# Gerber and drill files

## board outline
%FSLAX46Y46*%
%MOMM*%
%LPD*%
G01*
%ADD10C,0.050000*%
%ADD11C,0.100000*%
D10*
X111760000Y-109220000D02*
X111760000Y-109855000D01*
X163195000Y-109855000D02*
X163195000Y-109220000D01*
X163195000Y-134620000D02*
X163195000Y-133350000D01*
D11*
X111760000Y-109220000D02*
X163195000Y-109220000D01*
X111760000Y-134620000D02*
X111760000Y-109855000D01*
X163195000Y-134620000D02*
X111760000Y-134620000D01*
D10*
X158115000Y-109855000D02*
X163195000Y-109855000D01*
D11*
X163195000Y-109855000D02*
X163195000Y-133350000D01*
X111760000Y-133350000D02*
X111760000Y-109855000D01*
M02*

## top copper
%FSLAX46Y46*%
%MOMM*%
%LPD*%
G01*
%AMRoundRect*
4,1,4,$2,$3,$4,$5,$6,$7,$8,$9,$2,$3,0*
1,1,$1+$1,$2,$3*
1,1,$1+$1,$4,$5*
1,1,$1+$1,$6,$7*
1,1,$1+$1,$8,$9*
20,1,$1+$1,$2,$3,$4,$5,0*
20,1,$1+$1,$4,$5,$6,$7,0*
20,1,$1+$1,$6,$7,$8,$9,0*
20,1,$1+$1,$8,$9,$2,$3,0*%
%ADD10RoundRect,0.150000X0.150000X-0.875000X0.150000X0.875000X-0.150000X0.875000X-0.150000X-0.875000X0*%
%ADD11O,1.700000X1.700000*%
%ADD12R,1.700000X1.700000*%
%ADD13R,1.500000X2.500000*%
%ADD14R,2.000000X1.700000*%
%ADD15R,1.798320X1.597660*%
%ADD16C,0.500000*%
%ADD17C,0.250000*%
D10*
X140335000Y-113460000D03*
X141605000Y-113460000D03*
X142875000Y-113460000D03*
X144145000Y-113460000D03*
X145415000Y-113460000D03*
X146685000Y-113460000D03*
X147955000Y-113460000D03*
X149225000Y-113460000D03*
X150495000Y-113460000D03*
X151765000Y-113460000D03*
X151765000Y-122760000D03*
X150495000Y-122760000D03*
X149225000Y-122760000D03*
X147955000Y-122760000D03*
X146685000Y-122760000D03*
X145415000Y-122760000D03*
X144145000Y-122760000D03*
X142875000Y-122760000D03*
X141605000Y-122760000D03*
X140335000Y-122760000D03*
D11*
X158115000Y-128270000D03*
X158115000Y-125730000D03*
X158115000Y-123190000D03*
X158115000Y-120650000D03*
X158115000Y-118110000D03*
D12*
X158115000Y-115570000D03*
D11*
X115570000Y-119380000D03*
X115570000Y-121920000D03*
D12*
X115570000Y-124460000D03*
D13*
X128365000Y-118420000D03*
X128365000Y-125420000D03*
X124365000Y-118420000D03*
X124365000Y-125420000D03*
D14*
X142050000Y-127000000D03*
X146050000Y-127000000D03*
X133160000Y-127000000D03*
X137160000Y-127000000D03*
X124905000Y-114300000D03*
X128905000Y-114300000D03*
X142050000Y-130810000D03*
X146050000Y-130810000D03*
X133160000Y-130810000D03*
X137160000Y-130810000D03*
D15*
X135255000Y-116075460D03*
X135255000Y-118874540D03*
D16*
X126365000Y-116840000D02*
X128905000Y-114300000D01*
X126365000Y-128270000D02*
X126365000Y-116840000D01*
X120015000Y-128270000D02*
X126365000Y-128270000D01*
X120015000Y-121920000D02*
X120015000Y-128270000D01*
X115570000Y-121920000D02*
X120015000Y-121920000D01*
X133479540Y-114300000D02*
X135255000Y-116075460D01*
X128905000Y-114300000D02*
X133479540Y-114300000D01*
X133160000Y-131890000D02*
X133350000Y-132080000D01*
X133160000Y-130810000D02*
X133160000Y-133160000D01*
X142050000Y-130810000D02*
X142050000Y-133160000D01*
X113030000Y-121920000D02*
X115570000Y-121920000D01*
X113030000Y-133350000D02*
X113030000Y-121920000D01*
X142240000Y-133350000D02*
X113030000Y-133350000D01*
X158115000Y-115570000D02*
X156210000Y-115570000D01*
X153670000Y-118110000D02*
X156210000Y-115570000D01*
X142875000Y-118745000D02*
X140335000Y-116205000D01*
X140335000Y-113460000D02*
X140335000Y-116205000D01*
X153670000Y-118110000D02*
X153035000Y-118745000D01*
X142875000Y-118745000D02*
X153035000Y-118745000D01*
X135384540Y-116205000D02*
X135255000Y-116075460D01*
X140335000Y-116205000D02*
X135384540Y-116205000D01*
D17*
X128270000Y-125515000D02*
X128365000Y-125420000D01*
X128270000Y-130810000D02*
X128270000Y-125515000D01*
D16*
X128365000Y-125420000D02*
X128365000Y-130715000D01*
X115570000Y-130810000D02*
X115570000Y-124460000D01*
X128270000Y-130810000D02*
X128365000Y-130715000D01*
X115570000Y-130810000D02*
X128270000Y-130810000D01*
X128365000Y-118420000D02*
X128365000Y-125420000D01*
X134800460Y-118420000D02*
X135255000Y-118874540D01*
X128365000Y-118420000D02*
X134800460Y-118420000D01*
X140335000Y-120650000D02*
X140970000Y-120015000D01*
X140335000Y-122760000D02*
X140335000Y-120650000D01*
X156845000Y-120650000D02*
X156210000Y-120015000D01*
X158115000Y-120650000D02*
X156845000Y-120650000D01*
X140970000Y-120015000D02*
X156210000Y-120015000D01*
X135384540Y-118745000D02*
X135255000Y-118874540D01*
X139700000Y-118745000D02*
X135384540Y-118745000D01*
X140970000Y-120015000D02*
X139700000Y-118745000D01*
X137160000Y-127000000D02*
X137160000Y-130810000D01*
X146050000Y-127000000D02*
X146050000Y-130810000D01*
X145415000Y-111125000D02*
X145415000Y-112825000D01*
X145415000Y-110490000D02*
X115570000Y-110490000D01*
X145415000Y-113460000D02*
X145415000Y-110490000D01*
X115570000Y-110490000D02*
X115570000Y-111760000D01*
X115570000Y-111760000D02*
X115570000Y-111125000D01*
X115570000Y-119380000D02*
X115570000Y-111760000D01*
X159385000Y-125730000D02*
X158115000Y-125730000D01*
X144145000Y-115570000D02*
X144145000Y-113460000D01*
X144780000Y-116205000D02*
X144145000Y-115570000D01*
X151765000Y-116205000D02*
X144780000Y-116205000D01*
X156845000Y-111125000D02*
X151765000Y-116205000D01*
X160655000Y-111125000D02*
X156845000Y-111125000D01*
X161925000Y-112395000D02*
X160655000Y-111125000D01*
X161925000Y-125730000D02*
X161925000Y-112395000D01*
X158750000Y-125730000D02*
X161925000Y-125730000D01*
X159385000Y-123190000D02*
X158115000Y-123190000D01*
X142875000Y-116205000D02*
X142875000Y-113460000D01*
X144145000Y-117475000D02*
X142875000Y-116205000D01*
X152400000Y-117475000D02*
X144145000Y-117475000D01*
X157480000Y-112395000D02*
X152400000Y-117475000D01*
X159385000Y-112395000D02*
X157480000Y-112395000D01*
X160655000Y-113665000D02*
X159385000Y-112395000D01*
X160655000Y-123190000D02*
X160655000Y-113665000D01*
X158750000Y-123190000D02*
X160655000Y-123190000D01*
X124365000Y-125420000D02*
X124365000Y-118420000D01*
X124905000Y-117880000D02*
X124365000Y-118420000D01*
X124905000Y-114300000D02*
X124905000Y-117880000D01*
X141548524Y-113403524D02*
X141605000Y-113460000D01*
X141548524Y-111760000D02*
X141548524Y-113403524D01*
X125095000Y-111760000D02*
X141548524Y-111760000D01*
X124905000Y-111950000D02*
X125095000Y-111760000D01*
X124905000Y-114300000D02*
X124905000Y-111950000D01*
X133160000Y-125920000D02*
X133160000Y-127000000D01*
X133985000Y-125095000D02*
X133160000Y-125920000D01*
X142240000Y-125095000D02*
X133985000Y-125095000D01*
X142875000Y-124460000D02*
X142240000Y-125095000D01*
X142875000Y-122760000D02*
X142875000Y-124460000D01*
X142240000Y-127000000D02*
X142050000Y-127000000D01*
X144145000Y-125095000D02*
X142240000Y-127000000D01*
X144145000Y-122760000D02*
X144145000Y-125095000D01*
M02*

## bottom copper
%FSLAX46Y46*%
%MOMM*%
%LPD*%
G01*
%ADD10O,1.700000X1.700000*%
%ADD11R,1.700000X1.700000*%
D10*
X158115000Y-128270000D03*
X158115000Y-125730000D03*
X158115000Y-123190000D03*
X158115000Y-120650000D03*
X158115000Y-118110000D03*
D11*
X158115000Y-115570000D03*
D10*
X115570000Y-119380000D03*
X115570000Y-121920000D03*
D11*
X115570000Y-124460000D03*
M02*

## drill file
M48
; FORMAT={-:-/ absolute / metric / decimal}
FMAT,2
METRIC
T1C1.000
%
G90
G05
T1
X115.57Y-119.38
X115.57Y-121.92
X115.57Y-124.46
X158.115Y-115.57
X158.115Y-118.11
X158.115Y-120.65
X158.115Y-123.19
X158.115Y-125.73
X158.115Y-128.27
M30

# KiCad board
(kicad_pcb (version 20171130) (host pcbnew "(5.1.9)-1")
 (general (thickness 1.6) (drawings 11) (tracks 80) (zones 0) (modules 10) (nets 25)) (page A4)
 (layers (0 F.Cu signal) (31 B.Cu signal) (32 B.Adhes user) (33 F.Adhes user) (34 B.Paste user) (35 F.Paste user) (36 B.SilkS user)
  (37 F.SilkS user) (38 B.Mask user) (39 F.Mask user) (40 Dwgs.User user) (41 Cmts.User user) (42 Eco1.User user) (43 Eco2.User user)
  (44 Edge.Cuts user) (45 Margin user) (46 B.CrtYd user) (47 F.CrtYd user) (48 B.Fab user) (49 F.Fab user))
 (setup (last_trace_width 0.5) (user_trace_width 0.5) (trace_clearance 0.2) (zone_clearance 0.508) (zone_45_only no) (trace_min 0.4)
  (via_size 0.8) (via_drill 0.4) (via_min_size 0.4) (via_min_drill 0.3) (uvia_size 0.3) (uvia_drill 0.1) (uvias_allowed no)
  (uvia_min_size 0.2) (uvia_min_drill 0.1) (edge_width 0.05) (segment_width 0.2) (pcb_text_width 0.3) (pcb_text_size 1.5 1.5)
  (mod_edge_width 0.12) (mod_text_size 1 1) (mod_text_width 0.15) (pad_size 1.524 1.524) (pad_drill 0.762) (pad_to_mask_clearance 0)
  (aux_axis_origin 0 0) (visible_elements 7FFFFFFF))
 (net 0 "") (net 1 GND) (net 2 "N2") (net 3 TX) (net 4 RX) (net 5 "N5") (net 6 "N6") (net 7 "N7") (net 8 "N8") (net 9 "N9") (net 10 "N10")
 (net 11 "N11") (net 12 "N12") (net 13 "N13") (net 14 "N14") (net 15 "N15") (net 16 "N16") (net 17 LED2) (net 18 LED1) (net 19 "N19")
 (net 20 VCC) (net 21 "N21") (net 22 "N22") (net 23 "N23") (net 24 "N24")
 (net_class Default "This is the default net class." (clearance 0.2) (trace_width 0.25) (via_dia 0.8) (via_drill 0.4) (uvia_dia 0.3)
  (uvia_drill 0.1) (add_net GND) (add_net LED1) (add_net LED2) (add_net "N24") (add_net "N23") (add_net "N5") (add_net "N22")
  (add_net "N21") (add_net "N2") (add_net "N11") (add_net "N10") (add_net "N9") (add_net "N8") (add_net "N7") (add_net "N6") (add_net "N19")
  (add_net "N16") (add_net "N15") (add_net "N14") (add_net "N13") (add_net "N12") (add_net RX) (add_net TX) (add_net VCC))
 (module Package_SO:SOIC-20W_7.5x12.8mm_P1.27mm (layer F.Cu) (at 146.05 118.11 90)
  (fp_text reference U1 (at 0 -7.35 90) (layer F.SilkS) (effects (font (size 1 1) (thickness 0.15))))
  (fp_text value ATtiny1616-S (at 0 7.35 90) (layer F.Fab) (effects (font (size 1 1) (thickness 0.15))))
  (pad 20 smd roundrect (at 4.65 -5.715 90) (size 2.05 0.6) (layers F.Cu F.Paste F.Mask) (roundrect_rratio 0.25) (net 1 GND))
  (pad 19 smd roundrect (at 4.65 -4.445 90) (size 2.05 0.6) (layers F.Cu F.Paste F.Mask) (roundrect_rratio 0.25) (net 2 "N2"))
  (pad 18 smd roundrect (at 4.65 -3.175 90) (size 2.05 0.6) (layers F.Cu F.Paste F.Mask) (roundrect_rratio 0.25) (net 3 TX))
  (pad 17 smd roundrect (at 4.65 -1.905 90) (size 2.05 0.6) (layers F.Cu F.Paste F.Mask) (roundrect_rratio 0.25) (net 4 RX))
  (pad 16 smd roundrect (at 4.65 -0.635 90) (size 2.05 0.6) (layers F.Cu F.Paste F.Mask) (roundrect_rratio 0.25) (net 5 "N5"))
  (pad 15 smd roundrect (at 4.65 0.635 90) (size 2.05 0.6) (layers F.Cu F.Paste F.Mask) (roundrect_rratio 0.25) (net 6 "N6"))
  (pad 14 smd roundrect (at 4.65 1.905 90) (size 2.05 0.6) (layers F.Cu F.Paste F.Mask) (roundrect_rratio 0.25) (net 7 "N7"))
  (pad 13 smd roundrect (at 4.65 3.175 90) (size 2.05 0.6) (layers F.Cu F.Paste F.Mask) (roundrect_rratio 0.25) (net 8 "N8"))
  (pad 12 smd roundrect (at 4.65 4.445 90) (size 2.05 0.6) (layers F.Cu F.Paste F.Mask) (roundrect_rratio 0.25) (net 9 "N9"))
  (pad 11 smd roundrect (at 4.65 5.715 90) (size 2.05 0.6) (layers F.Cu F.Paste F.Mask) (roundrect_rratio 0.25) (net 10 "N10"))
  (pad 10 smd roundrect (at -4.65 5.715 90) (size 2.05 0.6) (layers F.Cu F.Paste F.Mask) (roundrect_rratio 0.25) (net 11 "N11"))
  (pad 9 smd roundrect (at -4.65 4.445 90) (size 2.05 0.6) (layers F.Cu F.Paste F.Mask) (roundrect_rratio 0.25) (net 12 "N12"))
  (pad 8 smd roundrect (at -4.65 3.175 90) (size 2.05 0.6) (layers F.Cu F.Paste F.Mask) (roundrect_rratio 0.25) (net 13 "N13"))
  (pad 7 smd roundrect (at -4.65 1.905 90) (size 2.05 0.6) (layers F.Cu F.Paste F.Mask) (roundrect_rratio 0.25) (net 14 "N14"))
  (pad 6 smd roundrect (at -4.65 0.635 90) (size 2.05 0.6) (layers F.Cu F.Paste F.Mask) (roundrect_rratio 0.25) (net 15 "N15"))
  (pad 5 smd roundrect (at -4.65 -0.635 90) (size 2.05 0.6) (layers F.Cu F.Paste F.Mask) (roundrect_rratio 0.25) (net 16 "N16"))
  (pad 4 smd roundrect (at -4.65 -1.905 90) (size 2.05 0.6) (layers F.Cu F.Paste F.Mask) (roundrect_rratio 0.25) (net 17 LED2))
  (pad 3 smd roundrect (at -4.65 -3.175 90) (size 2.05 0.6) (layers F.Cu F.Paste F.Mask) (roundrect_rratio 0.25) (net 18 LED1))
  (pad 2 smd roundrect (at -4.65 -4.445 90) (size 2.05 0.6) (layers F.Cu F.Paste F.Mask) (roundrect_rratio 0.25) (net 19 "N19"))
  (pad 1 smd roundrect (at -4.65 -5.715 90) (size 2.05 0.6) (layers F.Cu F.Paste F.Mask) (roundrect_rratio 0.25) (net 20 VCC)))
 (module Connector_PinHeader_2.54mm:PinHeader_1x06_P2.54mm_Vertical (layer F.Cu) (at 158.115 115.57)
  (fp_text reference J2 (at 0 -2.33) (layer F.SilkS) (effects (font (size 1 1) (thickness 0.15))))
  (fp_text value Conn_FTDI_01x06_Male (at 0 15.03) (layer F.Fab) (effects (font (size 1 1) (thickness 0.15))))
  (pad 6 thru_hole oval (at 0 12.7) (size 1.7 1.7) (drill 1) (layers *.Cu *.Mask) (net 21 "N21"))
  (pad 5 thru_hole oval (at 0 10.16) (size 1.7 1.7) (drill 1) (layers *.Cu *.Mask) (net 4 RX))
  (pad 4 thru_hole oval (at 0 7.62) (size 1.7 1.7) (drill 1) (layers *.Cu *.Mask) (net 3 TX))
  (pad 3 thru_hole oval (at 0 5.08) (size 1.7 1.7) (drill 1) (layers *.Cu *.Mask) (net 20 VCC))
  (pad 2 thru_hole oval (at 0 2.54) (size 1.7 1.7) (drill 1) (layers *.Cu *.Mask) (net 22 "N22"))
  (pad 1 thru_hole rect (at 0 0) (size 1.7 1.7) (drill 1) (layers *.Cu *.Mask) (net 1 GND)))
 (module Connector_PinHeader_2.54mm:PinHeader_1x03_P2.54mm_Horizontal (layer F.Cu) (at 115.57 124.46 180)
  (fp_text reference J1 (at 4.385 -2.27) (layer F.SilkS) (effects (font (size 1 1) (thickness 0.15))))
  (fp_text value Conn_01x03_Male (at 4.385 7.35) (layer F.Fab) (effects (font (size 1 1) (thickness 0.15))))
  (pad 3 thru_hole oval (at 0 5.08 180) (size 1.7 1.7) (drill 1) (layers *.Cu *.Mask) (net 5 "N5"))
  (pad 2 thru_hole oval (at 0 2.54 180) (size 1.7 1.7) (drill 1) (layers *.Cu *.Mask) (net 1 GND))
  (pad 1 thru_hole rect (at 0 0 180) (size 1.7 1.7) (drill 1) (layers *.Cu *.Mask) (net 20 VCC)))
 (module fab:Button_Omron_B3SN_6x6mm (layer F.Cu) (at 126.365 121.92 270)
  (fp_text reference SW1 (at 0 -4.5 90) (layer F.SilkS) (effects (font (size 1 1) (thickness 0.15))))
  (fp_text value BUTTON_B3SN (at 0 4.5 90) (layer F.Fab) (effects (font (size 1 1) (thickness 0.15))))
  (pad 1 smd rect (at -3.5 -2 270) (size 2.5 1.5) (layers F.Cu F.Paste F.Mask) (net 20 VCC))
  (pad 1 smd rect (at 3.5 -2 270) (size 2.5 1.5) (layers F.Cu F.Paste F.Mask) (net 20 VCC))
  (pad 2 smd rect (at -3.5 2 270) (size 2.5 1.5) (layers F.Cu F.Paste F.Mask) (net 2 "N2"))
  (pad 2 smd rect (at 3.5 2 270) (size 2.5 1.5) (layers F.Cu F.Paste F.Mask) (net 2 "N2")))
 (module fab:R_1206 (layer F.Cu) (at 144.05 127)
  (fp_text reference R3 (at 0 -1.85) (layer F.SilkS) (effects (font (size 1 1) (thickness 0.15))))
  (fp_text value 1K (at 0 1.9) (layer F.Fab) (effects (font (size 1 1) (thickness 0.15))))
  (pad 1 smd rect (at -2 0) (size 2 1.7) (layers F.Cu F.Paste F.Mask) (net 17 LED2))
  (pad 2 smd rect (at 2 0) (size 2 1.7) (layers F.Cu F.Paste F.Mask) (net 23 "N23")))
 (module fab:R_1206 (layer F.Cu) (at 135.16 127)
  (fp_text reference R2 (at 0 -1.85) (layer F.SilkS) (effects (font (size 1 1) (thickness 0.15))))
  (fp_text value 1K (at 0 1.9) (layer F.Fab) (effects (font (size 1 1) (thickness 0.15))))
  (pad 1 smd rect (at -2 0) (size 2 1.7) (layers F.Cu F.Paste F.Mask) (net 18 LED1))
  (pad 2 smd rect (at 2 0) (size 2 1.7) (layers F.Cu F.Paste F.Mask) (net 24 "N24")))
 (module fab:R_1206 (layer F.Cu) (at 126.905 114.3)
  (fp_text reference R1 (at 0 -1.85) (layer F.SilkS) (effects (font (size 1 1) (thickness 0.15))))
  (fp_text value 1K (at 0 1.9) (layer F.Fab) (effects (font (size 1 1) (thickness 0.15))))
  (pad 1 smd rect (at -2 0) (size 2 1.7) (layers F.Cu F.Paste F.Mask) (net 2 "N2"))
  (pad 2 smd rect (at 2 0) (size 2 1.7) (layers F.Cu F.Paste F.Mask) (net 1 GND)))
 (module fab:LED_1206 (layer F.Cu) (at 144.05 130.81)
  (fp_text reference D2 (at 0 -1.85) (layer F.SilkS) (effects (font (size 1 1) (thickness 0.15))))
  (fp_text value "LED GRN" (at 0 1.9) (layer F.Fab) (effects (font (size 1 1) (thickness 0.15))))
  (pad 1 smd rect (at -2 0) (size 2 1.7) (layers F.Cu F.Paste F.Mask) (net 1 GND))
  (pad 2 smd rect (at 2 0) (size 2 1.7) (layers F.Cu F.Paste F.Mask) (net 23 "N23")))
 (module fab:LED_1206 (layer F.Cu) (at 135.16 130.81)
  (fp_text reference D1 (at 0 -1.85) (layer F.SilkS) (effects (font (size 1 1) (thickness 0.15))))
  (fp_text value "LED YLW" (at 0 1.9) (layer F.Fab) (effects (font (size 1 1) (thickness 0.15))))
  (pad 1 smd rect (at -2 0) (size 2 1.7) (layers F.Cu F.Paste F.Mask) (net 1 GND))
  (pad 2 smd rect (at 2 0) (size 2 1.7) (layers F.Cu F.Paste F.Mask) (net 24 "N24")))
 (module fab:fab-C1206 (layer F.Cu) (at 135.255 117.475 90)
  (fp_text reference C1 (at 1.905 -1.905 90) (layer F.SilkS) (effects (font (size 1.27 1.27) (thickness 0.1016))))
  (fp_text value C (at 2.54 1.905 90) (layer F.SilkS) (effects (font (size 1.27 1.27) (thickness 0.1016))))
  (pad 2 smd rect (at 1.39954 0 90) (size 1.59766 1.79832) (layers F.Cu F.Paste F.Mask) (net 1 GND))
  (pad 1 smd rect (at -1.39954 0 90) (size 1.59766 1.79832) (layers F.Cu F.Paste F.Mask) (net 20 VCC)))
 (gr_line (start 111.76 109.22) (end 111.76 109.855) (layer Edge.Cuts) (width 0.05))
 (gr_line (start 163.195 109.855) (end 163.195 109.22) (layer Edge.Cuts) (width 0.05))
 (gr_line (start 163.195 134.62) (end 163.195 133.35) (layer Edge.Cuts) (width 0.05))
 (gr_line (start 111.76 109.22) (end 163.195 109.22) (layer Edge.Cuts) (width 0.1))
 (gr_line (start 111.76 134.62) (end 111.76 109.855) (layer Edge.Cuts) (width 0.1))
 (gr_line (start 163.195 134.62) (end 111.76 134.62) (layer Edge.Cuts) (width 0.1))
 (gr_line (start 158.115 109.855) (end 163.195 109.855) (layer Edge.Cuts) (width 0.05))
 (gr_line (start 163.195 109.855) (end 163.195 133.35) (layer Edge.Cuts) (width 0.1))
 (gr_line (start 111.76 133.35) (end 111.76 109.855) (layer Edge.Cuts) (width 0.1))
 (segment (start 126.365 116.84) (end 128.905 114.3) (width 0.5) (layer F.Cu) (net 1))
 (segment (start 126.365 128.27) (end 126.365 116.84) (width 0.5) (layer F.Cu) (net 1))
 (segment (start 120.015 128.27) (end 126.365 128.27) (width 0.5) (layer F.Cu) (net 1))
 (segment (start 120.015 121.92) (end 120.015 128.27) (width 0.5) (layer F.Cu) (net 1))
 (segment (start 115.57 121.92) (end 120.015 121.92) (width 0.5) (layer F.Cu) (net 1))
 (segment (start 133.47954 114.3) (end 135.255 116.07546) (width 0.5) (layer F.Cu) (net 1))
 (segment (start 128.905 114.3) (end 133.47954 114.3) (width 0.5) (layer F.Cu) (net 1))
 (segment (start 133.16 131.89) (end 133.35 132.08) (width 0.5) (layer F.Cu) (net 1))
 (segment (start 133.16 130.81) (end 133.16 133.16) (width 0.5) (layer F.Cu) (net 1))
 (segment (start 142.05 130.81) (end 142.05 133.16) (width 0.5) (layer F.Cu) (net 1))
 (segment (start 113.03 121.92) (end 115.57 121.92) (width 0.5) (layer F.Cu) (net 1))
 (segment (start 113.03 133.35) (end 113.03 121.92) (width 0.5) (layer F.Cu) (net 1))
 (segment (start 142.24 133.35) (end 113.03 133.35) (width 0.5) (layer F.Cu) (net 1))
 (segment (start 158.115 115.57) (end 156.21 115.57) (width 0.5) (layer F.Cu) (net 1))
 (segment (start 153.67 118.11) (end 156.21 115.57) (width 0.5) (layer F.Cu) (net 1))
 (segment (start 142.875 118.745) (end 140.335 116.205) (width 0.5) (layer F.Cu) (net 1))
 (segment (start 140.335 113.46) (end 140.335 116.205) (width 0.5) (layer F.Cu) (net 1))
 (segment (start 153.67 118.11) (end 153.035 118.745) (width 0.5) (layer F.Cu) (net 1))
 (segment (start 142.875 118.745) (end 153.035 118.745) (width 0.5) (layer F.Cu) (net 1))
 (segment (start 135.38454 116.205) (end 135.255 116.07546) (width 0.5) (layer F.Cu) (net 1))
 (segment (start 140.335 116.205) (end 135.38454 116.205) (width 0.5) (layer F.Cu) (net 1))
 (segment (start 128.27 125.515) (end 128.365 125.42) (width 0.25) (layer F.Cu) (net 20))
 (segment (start 128.27 130.81) (end 128.27 125.515) (width 0.25) (layer F.Cu) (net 20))
 (segment (start 128.365 125.42) (end 128.365 130.715) (width 0.5) (layer F.Cu) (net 20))
 (segment (start 115.57 130.81) (end 115.57 124.46) (width 0.5) (layer F.Cu) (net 20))
 (segment (start 128.27 130.81) (end 128.365 130.715) (width 0.5) (layer F.Cu) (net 20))
 (segment (start 115.57 130.81) (end 128.27 130.81) (width 0.5) (layer F.Cu) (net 20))
 (segment (start 128.365 118.42) (end 128.365 125.42) (width 0.5) (layer F.Cu) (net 20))
 (segment (start 134.80046 118.42) (end 135.255 118.87454) (width 0.5) (layer F.Cu) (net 20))
 (segment (start 128.365 118.42) (end 134.80046 118.42) (width 0.5) (layer F.Cu) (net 20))
 (segment (start 140.335 120.65) (end 140.97 120.015) (width 0.5) (layer F.Cu) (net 20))
 (segment (start 140.335 122.76) (end 140.335 120.65) (width 0.5) (layer F.Cu) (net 20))
 (segment (start 156.845 120.65) (end 156.21 120.015) (width 0.5) (layer F.Cu) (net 20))
 (segment (start 158.115 120.65) (end 156.845 120.65) (width 0.5) (layer F.Cu) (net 20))
 (segment (start 140.97 120.015) (end 156.21 120.015) (width 0.5) (layer F.Cu) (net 20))
 (segment (start 135.38454 118.745) (end 135.255 118.87454) (width 0.5) (layer F.Cu) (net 20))
 (segment (start 139.7 118.745) (end 135.38454 118.745) (width 0.5) (layer F.Cu) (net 20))
 (segment (start 140.97 120.015) (end 139.7 118.745) (width 0.5) (layer F.Cu) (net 20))
 (segment (start 137.16 127) (end 137.16 130.81) (width 0.5) (layer F.Cu) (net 24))
 (segment (start 146.05 127) (end 146.05 130.81) (width 0.5) (layer F.Cu) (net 23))
 (segment (start 145.415 111.125) (end 145.415 112.825) (width 0.5) (layer F.Cu) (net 5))
 (segment (start 145.415 110.49) (end 115.57 110.49) (width 0.5) (layer F.Cu) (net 5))
 (segment (start 145.415 113.46) (end 145.415 110.49) (width 0.5) (layer F.Cu) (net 5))
 (segment (start 115.57 110.49) (end 115.57 111.76) (width 0.5) (layer F.Cu) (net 5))
 (segment (start 115.57 111.76) (end 115.57 111.125) (width 0.5) (layer F.Cu) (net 5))
 (segment (start 115.57 119.38) (end 115.57 111.76) (width 0.5) (layer F.Cu) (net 5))
 (segment (start 159.385 125.73) (end 158.115 125.73) (width 0.5) (layer F.Cu) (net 4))
 (segment (start 144.145 115.57) (end 144.145 113.46) (width 0.5) (layer F.Cu) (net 4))
 (segment (start 144.78 116.205) (end 144.145 115.57) (width 0.5) (layer F.Cu) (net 4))
 (segment (start 151.765 116.205) (end 144.78 116.205) (width 0.5) (layer F.Cu) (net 4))
 (segment (start 156.845 111.125) (end 151.765 116.205) (width 0.5) (layer F.Cu) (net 4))
 (segment (start 160.655 111.125) (end 156.845 111.125) (width 0.5) (layer F.Cu) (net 4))
 (segment (start 161.925 112.395) (end 160.655 111.125) (width 0.5) (layer F.Cu) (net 4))
 (segment (start 161.925 125.73) (end 161.925 112.395) (width 0.5) (layer F.Cu) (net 4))
 (segment (start 158.75 125.73) (end 161.925 125.73) (width 0.5) (layer F.Cu) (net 4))
 (segment (start 159.385 123.19) (end 158.115 123.19) (width 0.5) (layer F.Cu) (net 3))
 (segment (start 142.875 116.205) (end 142.875 113.46) (width 0.5) (layer F.Cu) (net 3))
 (segment (start 144.145 117.475) (end 142.875 116.205) (width 0.5) (layer F.Cu) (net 3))
 (segment (start 152.4 117.475) (end 144.145 117.475) (width 0.5) (layer F.Cu) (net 3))
 (segment (start 157.48 112.395) (end 152.4 117.475) (width 0.5) (layer F.Cu) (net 3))
 (segment (start 159.385 112.395) (end 157.48 112.395) (width 0.5) (layer F.Cu) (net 3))
 (segment (start 160.655 113.665) (end 159.385 112.395) (width 0.5) (layer F.Cu) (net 3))
 (segment (start 160.655 123.19) (end 160.655 113.665) (width 0.5) (layer F.Cu) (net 3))
 (segment (start 158.75 123.19) (end 160.655 123.19) (width 0.5) (layer F.Cu) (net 3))
 (segment (start 124.365 125.42) (end 124.365 118.42) (width 0.5) (layer F.Cu) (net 2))
 (segment (start 124.905 117.88) (end 124.365 118.42) (width 0.5) (layer F.Cu) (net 2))
 (segment (start 124.905 114.3) (end 124.905 117.88) (width 0.5) (layer F.Cu) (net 2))
 (segment (start 141.548524 113.403524) (end 141.605 113.46) (width 0.5) (layer F.Cu) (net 2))
 (segment (start 141.548524 111.76) (end 141.548524 113.403524) (width 0.5) (layer F.Cu) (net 2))
 (segment (start 125.095 111.76) (end 141.548524 111.76) (width 0.5) (layer F.Cu) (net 2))
 (segment (start 124.905 111.95) (end 125.095 111.76) (width 0.5) (layer F.Cu) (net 2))
 (segment (start 124.905 114.3) (end 124.905 111.95) (width 0.5) (layer F.Cu) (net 2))
 (segment (start 133.16 125.92) (end 133.16 127) (width 0.5) (layer F.Cu) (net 18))
 (segment (start 133.985 125.095) (end 133.16 125.92) (width 0.5) (layer F.Cu) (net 18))
 (segment (start 142.24 125.095) (end 133.985 125.095) (width 0.5) (layer F.Cu) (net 18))
 (segment (start 142.875 124.46) (end 142.24 125.095) (width 0.5) (layer F.Cu) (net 18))
 (segment (start 142.875 122.76) (end 142.875 124.46) (width 0.5) (layer F.Cu) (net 18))
 (segment (start 142.24 127) (end 142.05 127) (width 0.5) (layer F.Cu) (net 17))
 (segment (start 144.145 125.095) (end 142.24 127) (width 0.5) (layer F.Cu) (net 17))
 (segment (start 144.145 122.76) (end 144.145 125.095) (width 0.5) (layer F.Cu) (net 17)))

